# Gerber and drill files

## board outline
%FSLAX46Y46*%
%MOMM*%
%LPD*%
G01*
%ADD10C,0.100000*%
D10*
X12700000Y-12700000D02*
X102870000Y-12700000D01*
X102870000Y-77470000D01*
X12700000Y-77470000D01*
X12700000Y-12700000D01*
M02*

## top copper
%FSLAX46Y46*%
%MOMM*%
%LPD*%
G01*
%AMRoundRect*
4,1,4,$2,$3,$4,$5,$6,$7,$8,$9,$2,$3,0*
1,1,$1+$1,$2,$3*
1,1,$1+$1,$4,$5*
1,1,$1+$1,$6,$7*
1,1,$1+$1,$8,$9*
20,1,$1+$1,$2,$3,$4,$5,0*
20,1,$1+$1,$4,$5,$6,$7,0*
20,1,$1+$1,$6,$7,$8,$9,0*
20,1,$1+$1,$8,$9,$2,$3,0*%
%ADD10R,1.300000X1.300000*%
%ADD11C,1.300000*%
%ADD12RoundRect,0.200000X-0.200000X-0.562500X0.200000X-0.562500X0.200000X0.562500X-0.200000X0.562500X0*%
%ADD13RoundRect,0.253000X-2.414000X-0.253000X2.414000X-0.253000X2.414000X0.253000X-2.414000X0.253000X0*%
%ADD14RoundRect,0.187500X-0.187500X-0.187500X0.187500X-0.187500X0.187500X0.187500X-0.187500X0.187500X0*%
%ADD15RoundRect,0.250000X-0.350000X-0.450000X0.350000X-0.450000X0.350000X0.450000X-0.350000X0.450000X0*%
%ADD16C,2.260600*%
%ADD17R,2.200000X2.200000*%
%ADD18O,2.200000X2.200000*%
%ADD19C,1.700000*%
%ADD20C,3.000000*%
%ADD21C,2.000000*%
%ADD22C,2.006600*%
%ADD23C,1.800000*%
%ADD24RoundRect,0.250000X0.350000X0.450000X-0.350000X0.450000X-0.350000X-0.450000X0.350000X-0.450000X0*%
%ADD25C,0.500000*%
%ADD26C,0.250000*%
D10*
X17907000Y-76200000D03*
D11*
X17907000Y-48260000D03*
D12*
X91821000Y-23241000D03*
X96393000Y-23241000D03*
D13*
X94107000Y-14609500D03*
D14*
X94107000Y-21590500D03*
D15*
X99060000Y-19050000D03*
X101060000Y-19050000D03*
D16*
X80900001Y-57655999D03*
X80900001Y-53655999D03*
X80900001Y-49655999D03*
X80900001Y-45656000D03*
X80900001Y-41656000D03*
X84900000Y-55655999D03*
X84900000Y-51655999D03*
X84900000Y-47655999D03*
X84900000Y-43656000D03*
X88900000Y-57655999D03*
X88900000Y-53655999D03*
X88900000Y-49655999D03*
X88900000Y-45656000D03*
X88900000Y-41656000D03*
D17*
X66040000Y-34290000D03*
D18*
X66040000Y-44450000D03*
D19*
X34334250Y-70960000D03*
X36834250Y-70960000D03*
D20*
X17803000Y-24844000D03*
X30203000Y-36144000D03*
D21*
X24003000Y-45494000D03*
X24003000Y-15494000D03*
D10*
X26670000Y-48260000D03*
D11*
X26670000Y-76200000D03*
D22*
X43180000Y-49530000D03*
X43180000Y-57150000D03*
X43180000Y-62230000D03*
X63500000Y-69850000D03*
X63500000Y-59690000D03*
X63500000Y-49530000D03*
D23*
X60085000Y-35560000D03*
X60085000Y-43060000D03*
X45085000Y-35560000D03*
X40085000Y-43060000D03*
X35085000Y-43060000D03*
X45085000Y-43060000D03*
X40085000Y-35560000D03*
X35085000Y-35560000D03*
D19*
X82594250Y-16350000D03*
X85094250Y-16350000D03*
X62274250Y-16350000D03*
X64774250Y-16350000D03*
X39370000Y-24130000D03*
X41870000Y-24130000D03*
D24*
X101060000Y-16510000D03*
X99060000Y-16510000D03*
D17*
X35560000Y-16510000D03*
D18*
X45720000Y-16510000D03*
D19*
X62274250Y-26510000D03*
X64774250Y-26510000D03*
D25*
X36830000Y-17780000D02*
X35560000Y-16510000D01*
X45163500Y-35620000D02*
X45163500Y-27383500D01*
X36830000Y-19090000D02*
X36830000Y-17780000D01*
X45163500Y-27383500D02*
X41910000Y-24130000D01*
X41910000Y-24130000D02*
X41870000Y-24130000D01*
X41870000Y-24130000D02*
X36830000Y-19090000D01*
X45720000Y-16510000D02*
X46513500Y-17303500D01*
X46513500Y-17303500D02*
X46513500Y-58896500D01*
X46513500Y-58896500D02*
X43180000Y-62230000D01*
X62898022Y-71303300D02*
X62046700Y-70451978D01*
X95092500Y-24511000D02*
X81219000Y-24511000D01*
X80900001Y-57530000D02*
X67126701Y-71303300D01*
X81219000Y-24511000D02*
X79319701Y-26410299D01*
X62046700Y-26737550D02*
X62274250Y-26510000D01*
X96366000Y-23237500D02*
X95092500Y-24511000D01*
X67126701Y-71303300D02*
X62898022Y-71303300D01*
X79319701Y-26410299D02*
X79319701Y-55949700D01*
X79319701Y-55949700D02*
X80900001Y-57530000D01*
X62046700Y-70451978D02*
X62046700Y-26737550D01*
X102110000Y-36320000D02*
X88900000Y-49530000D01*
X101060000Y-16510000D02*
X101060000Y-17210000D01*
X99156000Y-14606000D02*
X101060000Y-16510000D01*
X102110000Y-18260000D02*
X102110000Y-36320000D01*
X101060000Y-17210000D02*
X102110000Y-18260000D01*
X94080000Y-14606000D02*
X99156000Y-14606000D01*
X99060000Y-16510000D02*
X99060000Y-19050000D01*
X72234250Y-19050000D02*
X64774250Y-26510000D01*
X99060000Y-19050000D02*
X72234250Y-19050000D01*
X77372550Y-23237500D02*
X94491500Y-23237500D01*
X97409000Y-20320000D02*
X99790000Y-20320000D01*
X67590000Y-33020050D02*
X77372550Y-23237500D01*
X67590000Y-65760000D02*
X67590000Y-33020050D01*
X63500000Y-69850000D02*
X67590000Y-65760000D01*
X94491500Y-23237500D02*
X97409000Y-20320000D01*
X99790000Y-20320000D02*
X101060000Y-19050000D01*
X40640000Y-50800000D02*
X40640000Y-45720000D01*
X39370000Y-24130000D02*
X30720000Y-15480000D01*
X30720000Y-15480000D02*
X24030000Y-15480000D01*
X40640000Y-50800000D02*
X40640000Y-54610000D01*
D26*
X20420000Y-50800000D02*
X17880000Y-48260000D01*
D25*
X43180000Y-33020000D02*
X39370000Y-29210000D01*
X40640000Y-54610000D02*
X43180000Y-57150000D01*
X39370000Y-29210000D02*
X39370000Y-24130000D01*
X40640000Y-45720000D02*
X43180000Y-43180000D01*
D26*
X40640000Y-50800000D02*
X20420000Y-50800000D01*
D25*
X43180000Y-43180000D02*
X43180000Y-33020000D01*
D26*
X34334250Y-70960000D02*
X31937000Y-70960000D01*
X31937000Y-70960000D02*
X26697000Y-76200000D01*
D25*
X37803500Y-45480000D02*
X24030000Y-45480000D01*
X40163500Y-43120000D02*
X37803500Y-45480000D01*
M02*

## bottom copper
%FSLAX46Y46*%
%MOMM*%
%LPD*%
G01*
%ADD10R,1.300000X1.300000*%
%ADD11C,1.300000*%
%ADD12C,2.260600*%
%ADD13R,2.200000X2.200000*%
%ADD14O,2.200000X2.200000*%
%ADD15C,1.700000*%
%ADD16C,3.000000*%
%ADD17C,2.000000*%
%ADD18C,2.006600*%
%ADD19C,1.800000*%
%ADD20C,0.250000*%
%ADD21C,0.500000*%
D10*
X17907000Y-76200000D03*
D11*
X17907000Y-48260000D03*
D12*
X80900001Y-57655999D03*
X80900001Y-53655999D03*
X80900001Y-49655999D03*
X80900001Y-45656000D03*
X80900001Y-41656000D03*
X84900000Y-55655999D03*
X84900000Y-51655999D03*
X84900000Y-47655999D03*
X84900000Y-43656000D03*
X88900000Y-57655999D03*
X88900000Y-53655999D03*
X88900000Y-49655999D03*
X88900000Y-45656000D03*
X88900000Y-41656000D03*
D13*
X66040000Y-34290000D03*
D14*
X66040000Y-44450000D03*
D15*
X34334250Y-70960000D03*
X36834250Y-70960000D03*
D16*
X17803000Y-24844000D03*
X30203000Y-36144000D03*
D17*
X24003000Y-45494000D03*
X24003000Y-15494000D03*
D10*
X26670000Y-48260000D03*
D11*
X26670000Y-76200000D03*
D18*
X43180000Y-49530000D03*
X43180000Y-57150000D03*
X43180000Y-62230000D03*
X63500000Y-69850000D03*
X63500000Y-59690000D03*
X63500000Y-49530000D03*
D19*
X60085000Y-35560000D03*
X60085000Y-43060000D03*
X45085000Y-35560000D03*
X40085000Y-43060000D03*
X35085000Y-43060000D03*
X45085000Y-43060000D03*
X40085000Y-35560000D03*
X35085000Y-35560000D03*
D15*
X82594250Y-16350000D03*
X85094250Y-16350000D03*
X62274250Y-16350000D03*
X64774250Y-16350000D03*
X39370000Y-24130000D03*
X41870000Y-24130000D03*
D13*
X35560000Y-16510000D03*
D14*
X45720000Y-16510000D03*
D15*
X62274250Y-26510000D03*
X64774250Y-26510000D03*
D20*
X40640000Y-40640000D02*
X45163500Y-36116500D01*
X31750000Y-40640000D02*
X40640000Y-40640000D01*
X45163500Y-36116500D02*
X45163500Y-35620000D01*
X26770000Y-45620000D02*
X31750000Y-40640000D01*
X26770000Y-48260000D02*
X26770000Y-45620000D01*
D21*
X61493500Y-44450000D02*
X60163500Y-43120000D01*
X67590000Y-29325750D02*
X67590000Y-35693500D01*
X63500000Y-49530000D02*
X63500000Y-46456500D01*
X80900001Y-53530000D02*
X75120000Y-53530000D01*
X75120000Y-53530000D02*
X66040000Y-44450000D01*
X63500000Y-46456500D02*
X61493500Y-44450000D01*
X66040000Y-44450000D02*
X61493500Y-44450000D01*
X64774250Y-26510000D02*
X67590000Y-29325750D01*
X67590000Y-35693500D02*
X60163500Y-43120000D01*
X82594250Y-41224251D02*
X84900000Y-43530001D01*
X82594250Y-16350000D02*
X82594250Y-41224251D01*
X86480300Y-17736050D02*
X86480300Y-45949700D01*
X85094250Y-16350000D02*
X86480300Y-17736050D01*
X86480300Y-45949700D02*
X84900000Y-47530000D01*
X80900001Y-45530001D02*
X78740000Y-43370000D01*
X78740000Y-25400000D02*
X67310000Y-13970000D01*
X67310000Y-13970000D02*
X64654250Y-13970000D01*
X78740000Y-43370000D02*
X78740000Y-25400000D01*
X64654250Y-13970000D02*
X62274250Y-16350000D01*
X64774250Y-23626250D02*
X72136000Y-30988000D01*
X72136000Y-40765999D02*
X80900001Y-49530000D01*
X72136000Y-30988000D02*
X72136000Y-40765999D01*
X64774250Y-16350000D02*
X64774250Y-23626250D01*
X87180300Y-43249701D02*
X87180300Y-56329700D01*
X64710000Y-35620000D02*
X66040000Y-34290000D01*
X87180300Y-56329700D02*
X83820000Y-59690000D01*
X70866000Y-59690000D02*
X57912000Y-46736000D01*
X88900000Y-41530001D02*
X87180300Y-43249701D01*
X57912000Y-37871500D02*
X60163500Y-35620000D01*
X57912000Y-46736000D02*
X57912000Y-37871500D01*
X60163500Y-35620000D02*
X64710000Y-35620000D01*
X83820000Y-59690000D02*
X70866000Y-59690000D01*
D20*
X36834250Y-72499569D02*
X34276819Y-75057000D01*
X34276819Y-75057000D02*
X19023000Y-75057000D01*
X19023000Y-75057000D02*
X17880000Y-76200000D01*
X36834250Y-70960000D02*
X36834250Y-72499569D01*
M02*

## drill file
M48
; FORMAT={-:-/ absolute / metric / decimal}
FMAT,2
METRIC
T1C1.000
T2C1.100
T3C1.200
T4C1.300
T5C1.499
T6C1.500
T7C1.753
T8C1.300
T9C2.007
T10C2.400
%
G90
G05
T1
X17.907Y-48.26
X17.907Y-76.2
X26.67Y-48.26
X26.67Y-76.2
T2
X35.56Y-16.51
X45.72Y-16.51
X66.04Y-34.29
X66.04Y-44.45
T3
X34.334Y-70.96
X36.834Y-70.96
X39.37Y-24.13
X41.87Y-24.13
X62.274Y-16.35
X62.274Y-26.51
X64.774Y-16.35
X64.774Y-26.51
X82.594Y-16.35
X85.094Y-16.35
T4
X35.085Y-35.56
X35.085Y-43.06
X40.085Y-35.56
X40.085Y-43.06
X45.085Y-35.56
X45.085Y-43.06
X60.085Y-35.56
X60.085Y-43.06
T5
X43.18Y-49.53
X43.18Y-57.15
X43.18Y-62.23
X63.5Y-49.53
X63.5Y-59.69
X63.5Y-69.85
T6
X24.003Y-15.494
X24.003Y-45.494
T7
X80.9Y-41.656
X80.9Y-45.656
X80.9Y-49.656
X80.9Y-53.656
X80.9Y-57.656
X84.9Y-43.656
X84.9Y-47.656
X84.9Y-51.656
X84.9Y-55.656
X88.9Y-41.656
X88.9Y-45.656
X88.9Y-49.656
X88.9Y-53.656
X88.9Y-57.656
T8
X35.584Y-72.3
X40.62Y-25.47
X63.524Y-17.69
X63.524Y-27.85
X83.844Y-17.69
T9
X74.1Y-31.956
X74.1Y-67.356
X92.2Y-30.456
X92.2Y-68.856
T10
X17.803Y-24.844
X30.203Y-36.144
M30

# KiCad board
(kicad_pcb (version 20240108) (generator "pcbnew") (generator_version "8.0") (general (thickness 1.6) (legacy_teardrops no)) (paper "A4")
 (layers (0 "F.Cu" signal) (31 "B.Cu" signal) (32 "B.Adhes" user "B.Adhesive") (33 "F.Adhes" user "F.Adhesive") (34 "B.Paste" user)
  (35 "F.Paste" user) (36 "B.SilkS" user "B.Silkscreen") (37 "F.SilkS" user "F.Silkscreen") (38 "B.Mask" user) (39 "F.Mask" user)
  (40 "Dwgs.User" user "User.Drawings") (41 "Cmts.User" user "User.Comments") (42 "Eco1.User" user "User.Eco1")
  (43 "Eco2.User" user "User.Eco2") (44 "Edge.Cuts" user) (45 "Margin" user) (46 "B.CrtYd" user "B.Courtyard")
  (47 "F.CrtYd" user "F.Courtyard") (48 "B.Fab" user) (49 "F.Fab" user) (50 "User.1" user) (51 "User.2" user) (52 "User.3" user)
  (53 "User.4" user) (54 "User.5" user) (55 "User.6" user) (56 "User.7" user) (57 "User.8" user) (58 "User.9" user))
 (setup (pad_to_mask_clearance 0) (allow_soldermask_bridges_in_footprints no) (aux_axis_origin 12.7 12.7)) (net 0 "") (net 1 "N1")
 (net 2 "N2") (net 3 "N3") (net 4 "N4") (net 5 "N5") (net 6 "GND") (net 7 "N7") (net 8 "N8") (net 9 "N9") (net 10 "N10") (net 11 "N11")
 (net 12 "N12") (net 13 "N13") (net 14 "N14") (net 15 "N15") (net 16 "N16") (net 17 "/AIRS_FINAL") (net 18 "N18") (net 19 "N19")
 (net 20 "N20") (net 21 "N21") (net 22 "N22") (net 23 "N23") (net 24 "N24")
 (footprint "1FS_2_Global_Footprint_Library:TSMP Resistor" (layer "F.Cu") (at 17.907 62.103 90)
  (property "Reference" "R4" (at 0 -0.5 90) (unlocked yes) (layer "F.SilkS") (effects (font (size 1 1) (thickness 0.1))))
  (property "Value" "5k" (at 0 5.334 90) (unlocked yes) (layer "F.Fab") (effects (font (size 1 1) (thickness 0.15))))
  (pad "1" thru_hole rect (at -14.097 0 90) (size 1.3 1.3) (drill 1) (layers "*.Cu" "*.Mask") (remove_unused_layers no) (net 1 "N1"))
  (pad "2" thru_hole circle (at 13.843 0 90) (size 1.3 1.3) (drill 1) (layers "*.Cu" "*.Mask") (remove_unused_layers no) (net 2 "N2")))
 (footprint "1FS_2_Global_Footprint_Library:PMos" (layer "F.Cu") (at 94.182 18.5485)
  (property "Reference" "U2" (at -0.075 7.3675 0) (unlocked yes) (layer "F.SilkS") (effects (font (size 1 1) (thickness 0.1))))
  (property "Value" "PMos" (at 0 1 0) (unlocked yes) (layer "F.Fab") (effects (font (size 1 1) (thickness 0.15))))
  (pad "1" smd roundrect (at -2.361 4.6925) (size 0.8 1.525) (layers "F.Cu" "F.Paste" "F.Mask") (roundrect_rratio 0.25) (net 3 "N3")
   (thermal_bridge_angle 45))
  (pad "2" smd roundrect (at 2.211 4.6925) (size 0.8 1.525) (layers "F.Cu" "F.Paste" "F.Mask") (roundrect_rratio 0.25) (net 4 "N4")
   (thermal_bridge_angle 45))
  (pad "3" smd roundrect (at -0.075 -3.939) (size 5.334 1.012) (layers "F.Cu" "F.Paste" "F.Mask") (roundrect_rratio 0.25) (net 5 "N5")
   (thermal_bridge_angle 45))
  (pad "4" smd roundrect (at -0.075 3.042) (size 0.75 0.75) (layers "F.Cu" "F.Paste" "F.Mask") (roundrect_rratio 0.25)
   (thermal_bridge_angle 45)))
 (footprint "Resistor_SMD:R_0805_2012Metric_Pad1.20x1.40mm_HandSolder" (layer "F.Cu") (at 100.06 19.05)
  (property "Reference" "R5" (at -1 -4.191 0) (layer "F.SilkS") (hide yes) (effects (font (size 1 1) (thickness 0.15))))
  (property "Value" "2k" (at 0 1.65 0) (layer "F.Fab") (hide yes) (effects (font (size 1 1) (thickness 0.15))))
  (pad "1" smd roundrect (at -1 0) (size 1.2 1.4) (layers "F.Cu" "F.Paste" "F.Mask") (roundrect_rratio 0.2083333333) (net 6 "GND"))
  (pad "2" smd roundrect (at 1 0) (size 1.2 1.4) (layers "F.Cu" "F.Paste" "F.Mask") (roundrect_rratio 0.2083333333) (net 3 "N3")))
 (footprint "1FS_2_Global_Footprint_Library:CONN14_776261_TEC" (layer "F.Cu") (at 83.9 50.9105 90)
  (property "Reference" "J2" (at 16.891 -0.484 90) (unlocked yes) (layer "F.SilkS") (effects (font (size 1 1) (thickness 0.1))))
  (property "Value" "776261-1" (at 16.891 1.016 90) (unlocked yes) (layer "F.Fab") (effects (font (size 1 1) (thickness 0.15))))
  (pad "" np_thru_hole circle (at -17.945499 8.300001 90) (size 2.0066 2.0066) (drill 2.0066) (layers "*.Cu" "*.Mask"))
  (pad "" np_thru_hole circle (at -16.445503 -9.799999 90) (size 2.0066 2.0066) (drill 2.0066) (layers "*.Cu" "*.Mask"))
  (pad "" np_thru_hole circle (at 18.954504 -9.799999 90) (size 2.0066 2.0066) (drill 2.0066) (layers "*.Cu" "*.Mask"))
  (pad "" np_thru_hole circle (at 20.454501 8.300001 90) (size 2.0066 2.0066) (drill 2.0066) (layers "*.Cu" "*.Mask"))
  (pad "1" thru_hole circle (at -6.745499 -2.999999 90) (size 2.2606 2.2606) (drill 1.7526) (layers "*.Cu" "*.Mask")
   (remove_unused_layers no) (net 4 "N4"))
  (pad "2" thru_hole circle (at -2.745499 -2.999999 90) (size 2.2606 2.2606) (drill 1.7526) (layers "*.Cu" "*.Mask")
   (remove_unused_layers no) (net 6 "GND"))
  (pad "3" thru_hole circle (at 1.254501 -2.999999 90) (size 2.2606 2.2606) (drill 1.7526) (layers "*.Cu" "*.Mask")
   (remove_unused_layers no) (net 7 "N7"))
  (pad "4" thru_hole circle (at 5.2545 -2.999999 90) (size 2.2606 2.2606) (drill 1.7526) (layers "*.Cu" "*.Mask") (remove_unused_layers no)
   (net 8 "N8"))
  (pad "5" thru_hole circle (at 9.2545 -2.999999 90) (size 2.2606 2.2606) (drill 1.7526) (layers "*.Cu" "*.Mask") (remove_unused_layers no)
   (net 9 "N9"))
  (pad "6" thru_hole circle (at -4.745499 1 90) (size 2.2606 2.2606) (drill 1.7526) (layers "*.Cu" "*.Mask") (remove_unused_layers no)
   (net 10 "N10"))
  (pad "7" thru_hole circle (at -0.745499 1 90) (size 2.2606 2.2606) (drill 1.7526) (layers "*.Cu" "*.Mask") (remove_unused_layers no)
   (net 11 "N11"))
  (pad "8" thru_hole circle (at 3.254501 1 90) (size 2.2606 2.2606) (drill 1.7526) (layers "*.Cu" "*.Mask") (remove_unused_layers no)
   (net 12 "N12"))
  (pad "9" thru_hole circle (at 7.2545 1 90) (size 2.2606 2.2606) (drill 1.7526) (layers "*.Cu" "*.Mask") (remove_unused_layers no)
   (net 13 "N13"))
  (pad "10" thru_hole circle (at -6.745499 5 90) (size 2.2606 2.2606) (drill 1.7526) (layers "*.Cu" "*.Mask") (remove_unused_layers no)
   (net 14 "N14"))
  (pad "11" thru_hole circle (at -2.745499 5 90) (size 2.2606 2.2606) (drill 1.7526) (layers "*.Cu" "*.Mask") (remove_unused_layers no)
   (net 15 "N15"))
  (pad "12" thru_hole circle (at 1.254501 5 90) (size 2.2606 2.2606) (drill 1.7526) (layers "*.Cu" "*.Mask") (remove_unused_layers no)
   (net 5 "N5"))
  (pad "13" thru_hole circle (at 5.2545 5 90) (size 2.2606 2.2606) (drill 1.7526) (layers "*.Cu" "*.Mask") (remove_unused_layers no)
   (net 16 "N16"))
  (pad "14" thru_hole circle (at 9.2545 5 90) (size 2.2606 2.2606) (drill 1.7526) (layers "*.Cu" "*.Mask") (remove_unused_layers no)
   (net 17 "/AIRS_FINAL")))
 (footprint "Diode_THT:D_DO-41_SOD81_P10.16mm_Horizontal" (layer "F.Cu") (at 66.04 34.29 -90)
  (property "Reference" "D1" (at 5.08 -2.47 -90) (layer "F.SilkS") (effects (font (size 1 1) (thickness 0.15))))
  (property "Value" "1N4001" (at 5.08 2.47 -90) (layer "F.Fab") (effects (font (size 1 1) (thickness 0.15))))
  (pad "1" thru_hole rect (at 0 0 270) (size 2.2 2.2) (drill 1.1) (layers "*.Cu" "*.Mask") (remove_unused_layers no) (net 17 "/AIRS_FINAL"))
  (pad "2" thru_hole oval (at 10.16 0 270) (size 2.2 2.2) (drill 1.1) (layers "*.Cu" "*.Mask") (remove_unused_layers no) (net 6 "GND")))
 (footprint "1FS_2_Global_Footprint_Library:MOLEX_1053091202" (layer "F.Cu") (at 34.33425 70.96)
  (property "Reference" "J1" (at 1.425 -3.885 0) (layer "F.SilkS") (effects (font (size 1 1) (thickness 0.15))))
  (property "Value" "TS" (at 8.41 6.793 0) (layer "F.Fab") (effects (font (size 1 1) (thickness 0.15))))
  (pad "" np_thru_hole circle (at 1.25 1.34) (size 1.3 1.3) (drill 1.3) (layers "*.Cu" "*.Mask"))
  (pad "1" thru_hole circle (at 0 0) (size 1.7 1.7) (drill 1.2) (layers "*.Cu") (remove_unused_layers no) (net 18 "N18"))
  (pad "2" thru_hole circle (at 2.5 0) (size 1.7 1.7) (drill 1.2) (layers "*.Cu") (remove_unused_layers no) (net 1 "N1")))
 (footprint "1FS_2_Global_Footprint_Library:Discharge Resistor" (layer "F.Cu") (at 24.003 30.357 -90)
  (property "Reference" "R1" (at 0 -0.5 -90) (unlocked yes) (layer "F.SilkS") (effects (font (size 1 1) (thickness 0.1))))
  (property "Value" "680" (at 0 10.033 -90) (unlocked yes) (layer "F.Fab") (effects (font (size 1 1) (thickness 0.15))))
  (pad "" np_thru_hole circle (at -5.513 6.2 270) (size 3 3) (drill 2.4) (layers "F&B.Cu" "*.Mask"))
  (pad "" np_thru_hole circle (at 5.787 -6.2 270) (size 3 3) (drill 2.4) (layers "F&B.Cu" "*.Mask"))
  (pad "1" thru_hole circle (at 15.137 0 270) (size 2 2) (drill 1.5) (layers "*.Cu" "*.Mask") (remove_unused_layers no) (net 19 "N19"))
  (pad "2" thru_hole circle (at -14.863 0 270) (size 2 2) (drill 1.5) (layers "*.Cu" "*.Mask") (remove_unused_layers no) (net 2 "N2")))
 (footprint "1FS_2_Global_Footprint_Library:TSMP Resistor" (layer "F.Cu") (at 26.67 62.357 -90)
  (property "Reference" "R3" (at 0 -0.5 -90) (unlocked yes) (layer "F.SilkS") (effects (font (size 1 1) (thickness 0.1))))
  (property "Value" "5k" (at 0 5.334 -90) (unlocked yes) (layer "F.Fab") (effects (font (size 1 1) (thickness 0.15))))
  (pad "1" thru_hole rect (at -14.097 0 270) (size 1.3 1.3) (drill 1) (layers "*.Cu" "*.Mask") (remove_unused_layers no) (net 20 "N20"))
  (pad "2" thru_hole circle (at 13.843 0 270) (size 1.3 1.3) (drill 1) (layers "*.Cu" "*.Mask") (remove_unused_layers no) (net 18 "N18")))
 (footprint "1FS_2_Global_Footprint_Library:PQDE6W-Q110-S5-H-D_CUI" (layer "F.Cu") (at 43.18 49.53)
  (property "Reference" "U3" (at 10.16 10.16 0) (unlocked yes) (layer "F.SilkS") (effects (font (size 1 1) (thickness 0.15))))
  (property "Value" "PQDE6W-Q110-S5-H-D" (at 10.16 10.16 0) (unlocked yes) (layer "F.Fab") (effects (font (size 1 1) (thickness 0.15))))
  (pad "1" thru_hole circle (at 0 0) (size 2.0066 2.0066) (drill 1.4986) (layers "*.Cu" "*.Mask") (remove_unused_layers no) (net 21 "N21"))
  (pad "2" thru_hole circle (at 0 7.62) (size 2.0066 2.0066) (drill 1.4986) (layers "*.Cu" "*.Mask") (remove_unused_layers no) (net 2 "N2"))
  (pad "3" thru_hole circle (at 0 12.7) (size 2.0066 2.0066) (drill 1.4986) (layers "*.Cu" "*.Mask") (remove_unused_layers no)
   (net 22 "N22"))
  (pad "4" thru_hole circle (at 20.32 20.32) (size 2.0066 2.0066) (drill 1.4986) (layers "*.Cu" "*.Mask") (remove_unused_layers no)
   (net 3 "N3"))
  (pad "5" thru_hole circle (at 20.32 10.16) (size 2.0066 2.0066) (drill 1.4986) (layers "*.Cu" "*.Mask") (remove_unused_layers no)
   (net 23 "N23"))
  (pad "6" thru_hole circle (at 20.32 0) (size 2.0066 2.0066) (drill 1.4986) (layers "*.Cu" "*.Mask") (remove_unused_layers no)
   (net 6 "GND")))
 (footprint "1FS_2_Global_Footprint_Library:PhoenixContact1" (layer "F.Cu") (at 44.5 39.41 -90)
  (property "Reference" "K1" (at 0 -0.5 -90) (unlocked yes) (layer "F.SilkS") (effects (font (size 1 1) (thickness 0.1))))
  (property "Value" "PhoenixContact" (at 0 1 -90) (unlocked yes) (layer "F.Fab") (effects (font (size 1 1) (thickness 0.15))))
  (pad "1" thru_hole circle (at -3.85 -15.585 270) (size 1.8 1.8) (drill 1.3) (layers "*.Cu" "*.Mask") (remove_unused_layers no)
   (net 17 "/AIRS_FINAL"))
  (pad "2" thru_hole circle (at 3.65 -15.585 270) (size 1.8 1.8) (drill 1.3) (layers "*.Cu" "*.Mask") (remove_unused_layers no)
   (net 6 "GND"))
  (pad "3" thru_hole circle (at -3.85 -0.585 270) (size 1.8 1.8) (drill 1.3) (layers "*.Cu" "*.Mask") (remove_unused_layers no)
   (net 20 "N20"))
  (pad "4" thru_hole circle (at 3.65 4.415 270) (size 1.8 1.8) (drill 1.3) (layers "*.Cu" "*.Mask") (remove_unused_layers no) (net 19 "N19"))
  (pad "5" thru_hole circle (at 3.65 9.415 270) (size 1.8 1.8) (drill 1.3) (layers "*.Cu" "*.Mask") (remove_unused_layers no) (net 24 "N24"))
  (pad "6" thru_hole circle (at 3.65 -0.585 270) (size 1.8 1.8) (drill 1.3) (layers "*.Cu" "*.Mask") (remove_unused_layers no))
  (pad "7" thru_hole circle (at -3.85 4.415 270) (size 1.8 1.8) (drill 1.3) (layers "*.Cu" "*.Mask") (remove_unused_layers no))
  (pad "8" thru_hole circle (at -3.85 9.415 270) (size 1.8 1.8) (drill 1.3) (layers "*.Cu" "*.Mask") (remove_unused_layers no)))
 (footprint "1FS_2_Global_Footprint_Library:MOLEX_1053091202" (layer "F.Cu") (at 82.59425 16.35)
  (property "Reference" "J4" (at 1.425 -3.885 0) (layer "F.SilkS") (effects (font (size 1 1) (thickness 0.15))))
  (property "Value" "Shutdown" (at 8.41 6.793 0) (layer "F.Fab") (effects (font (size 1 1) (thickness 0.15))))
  (pad "" np_thru_hole circle (at 1.25 1.34) (size 1.3 1.3) (drill 1.3) (layers "*.Cu" "*.Mask"))
  (pad "1" thru_hole circle (at 0 0) (size 1.7 1.7) (drill 1.2) (layers "*.Cu") (remove_unused_layers no) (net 13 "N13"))
  (pad "2" thru_hole circle (at 2.5 0) (size 1.7 1.7) (drill 1.2) (layers "*.Cu") (remove_unused_layers no) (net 12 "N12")))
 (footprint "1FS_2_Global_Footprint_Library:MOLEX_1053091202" (layer "F.Cu") (at 62.27425 16.35)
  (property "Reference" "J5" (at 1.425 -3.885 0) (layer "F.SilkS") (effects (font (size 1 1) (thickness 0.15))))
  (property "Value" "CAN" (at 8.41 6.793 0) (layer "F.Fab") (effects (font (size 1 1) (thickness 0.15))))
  (pad "" np_thru_hole circle (at 1.25 1.34) (size 1.3 1.3) (drill 1.3) (layers "*.Cu" "*.Mask"))
  (pad "1" thru_hole circle (at 0 0) (size 1.7 1.7) (drill 1.2) (layers "*.Cu") (remove_unused_layers no) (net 8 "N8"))
  (pad "2" thru_hole circle (at 2.5 0) (size 1.7 1.7) (drill 1.2) (layers "*.Cu") (remove_unused_layers no) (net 7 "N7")))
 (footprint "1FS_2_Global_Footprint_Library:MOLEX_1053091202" (layer "F.Cu") (at 39.37 24.13)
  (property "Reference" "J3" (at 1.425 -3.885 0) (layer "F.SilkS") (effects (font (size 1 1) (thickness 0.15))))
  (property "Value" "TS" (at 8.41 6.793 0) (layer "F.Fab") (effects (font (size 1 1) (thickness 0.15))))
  (pad "" np_thru_hole circle (at 1.25 1.34) (size 1.3 1.3) (drill 1.3) (layers "*.Cu" "*.Mask"))
  (pad "1" thru_hole circle (at 0 0) (size 1.7 1.7) (drill 1.2) (layers "*.Cu") (remove_unused_layers no) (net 2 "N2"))
  (pad "2" thru_hole circle (at 2.5 0) (size 1.7 1.7) (drill 1.2) (layers "*.Cu") (remove_unused_layers no) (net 20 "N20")))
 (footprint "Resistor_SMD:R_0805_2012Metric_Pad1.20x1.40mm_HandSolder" (layer "F.Cu") (at 100.06 16.51 180)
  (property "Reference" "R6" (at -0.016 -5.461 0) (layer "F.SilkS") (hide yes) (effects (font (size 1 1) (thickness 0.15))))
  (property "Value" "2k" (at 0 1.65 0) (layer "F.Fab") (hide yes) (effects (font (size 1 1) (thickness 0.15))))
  (pad "1" smd roundrect (at -1 0 180) (size 1.2 1.4) (layers "F.Cu" "F.Paste" "F.Mask") (roundrect_rratio 0.2083333333) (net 5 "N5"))
  (pad "2" smd roundrect (at 1 0 180) (size 1.2 1.4) (layers "F.Cu" "F.Paste" "F.Mask") (roundrect_rratio 0.2083333333) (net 6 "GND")))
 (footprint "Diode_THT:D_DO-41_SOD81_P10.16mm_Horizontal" (layer "F.Cu") (at 35.56 16.51)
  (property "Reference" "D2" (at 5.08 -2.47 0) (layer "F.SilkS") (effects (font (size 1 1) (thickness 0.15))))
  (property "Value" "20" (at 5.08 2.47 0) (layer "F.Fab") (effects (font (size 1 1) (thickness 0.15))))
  (pad "1" thru_hole rect (at 0 0) (size 2.2 2.2) (drill 1.1) (layers "*.Cu" "*.Mask") (remove_unused_layers no) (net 20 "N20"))
  (pad "2" thru_hole oval (at 10.16 0) (size 2.2 2.2) (drill 1.1) (layers "*.Cu" "*.Mask") (remove_unused_layers no) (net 22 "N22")))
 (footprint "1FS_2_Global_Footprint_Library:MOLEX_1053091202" (layer "F.Cu") (at 62.27425 26.51)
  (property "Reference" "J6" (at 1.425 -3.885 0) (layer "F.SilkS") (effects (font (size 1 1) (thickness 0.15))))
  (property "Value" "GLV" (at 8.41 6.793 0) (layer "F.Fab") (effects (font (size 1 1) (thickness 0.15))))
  (pad "" np_thru_hole circle (at 1.25 1.34) (size 1.3 1.3) (drill 1.3) (layers "*.Cu" "*.Mask"))
  (pad "1" thru_hole circle (at 0 0) (size 1.7 1.7) (drill 1.2) (layers "*.Cu") (remove_unused_layers no) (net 4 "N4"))
  (pad "2" thru_hole circle (at 2.5 0) (size 1.7 1.7) (drill 1.2) (layers "*.Cu") (remove_unused_layers no) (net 6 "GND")))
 (gr_rect (start 12.7 12.7) (end 102.87 77.47) (stroke (width 0.1) (type default)) (fill none) (layer "Edge.Cuts"))
 (segment (start 36.83 17.78) (end 35.56 16.51) (width 0.5) (layer "F.Cu") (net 20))
 (segment (start 45.1635 35.62) (end 45.1635 27.3835) (width 0.5) (layer "F.Cu") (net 20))
 (segment (start 36.83 19.09) (end 36.83 17.78) (width 0.5) (layer "F.Cu") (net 20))
 (segment (start 45.1635 27.3835) (end 41.91 24.13) (width 0.5) (layer "F.Cu") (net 20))
 (segment (start 41.91 24.13) (end 41.87 24.13) (width 0.5) (layer "F.Cu") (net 20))
 (segment (start 41.87 24.13) (end 36.83 19.09) (width 0.5) (layer "F.Cu") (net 20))
 (segment (start 40.64 40.64) (end 45.1635 36.1165) (width 0.25) (layer "B.Cu") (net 20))
 (segment (start 31.75 40.64) (end 40.64 40.64) (width 0.25) (layer "B.Cu") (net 20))
 (segment (start 45.1635 36.1165) (end 45.1635 35.62) (width 0.25) (layer "B.Cu") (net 20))
 (segment (start 26.77 45.62) (end 31.75 40.64) (width 0.25) (layer "B.Cu") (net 20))
 (segment (start 26.77 48.26) (end 26.77 45.62) (width 0.25) (layer "B.Cu") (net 20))
 (segment (start 45.72 16.51) (end 46.5135 17.3035) (width 0.5) (layer "F.Cu") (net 22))
 (segment (start 46.5135 17.3035) (end 46.5135 58.8965) (width 0.5) (layer "F.Cu") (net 22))
 (segment (start 46.5135 58.8965) (end 43.18 62.23) (width 0.5) (layer "F.Cu") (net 22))
 (segment (start 62.898022 71.3033) (end 62.0467 70.451978) (width 0.5) (layer "F.Cu") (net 4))
 (segment (start 95.0925 24.511) (end 81.219 24.511) (width 0.5) (layer "F.Cu") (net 4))
 (segment (start 80.900001 57.53) (end 67.126701 71.3033) (width 0.5) (layer "F.Cu") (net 4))
 (segment (start 81.219 24.511) (end 79.319701 26.410299) (width 0.5) (layer "F.Cu") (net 4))
 (segment (start 62.0467 26.73755) (end 62.27425 26.51) (width 0.5) (layer "F.Cu") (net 4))
 (segment (start 96.366 23.2375) (end 95.0925 24.511) (width 0.5) (layer "F.Cu") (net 4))
 (segment (start 67.126701 71.3033) (end 62.898022 71.3033) (width 0.5) (layer "F.Cu") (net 4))
 (segment (start 79.319701 26.410299) (end 79.319701 55.9497) (width 0.5) (layer "F.Cu") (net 4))
 (segment (start 79.319701 55.9497) (end 80.900001 57.53) (width 0.5) (layer "F.Cu") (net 4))
 (segment (start 62.0467 70.451978) (end 62.0467 26.73755) (width 0.5) (layer "F.Cu") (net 4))
 (segment (start 102.11 36.32) (end 88.9 49.53) (width 0.5) (layer "F.Cu") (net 5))
 (segment (start 101.06 16.51) (end 101.06 17.21) (width 0.5) (layer "F.Cu") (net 5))
 (segment (start 99.156 14.606) (end 101.06 16.51) (width 0.5) (layer "F.Cu") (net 5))
 (segment (start 102.11 18.26) (end 102.11 36.32) (width 0.5) (layer "F.Cu") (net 5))
 (segment (start 101.06 17.21) (end 102.11 18.26) (width 0.5) (layer "F.Cu") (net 5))
 (segment (start 94.08 14.606) (end 99.156 14.606) (width 0.5) (layer "F.Cu") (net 5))
 (segment (start 99.06 16.51) (end 99.06 19.05) (width 0.5) (layer "F.Cu") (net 6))
 (segment (start 72.23425 19.05) (end 64.77425 26.51) (width 0.5) (layer "F.Cu") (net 6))
 (segment (start 99.06 19.05) (end 72.23425 19.05) (width 0.5) (layer "F.Cu") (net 6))
 (segment (start 61.4935 44.45) (end 60.1635 43.12) (width 0.5) (layer "B.Cu") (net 6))
 (segment (start 67.59 29.32575) (end 67.59 35.6935) (width 0.5) (layer "B.Cu") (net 6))
 (segment (start 63.5 49.53) (end 63.5 46.4565) (width 0.5) (layer "B.Cu") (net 6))
 (segment (start 80.900001 53.53) (end 75.12 53.53) (width 0.5) (layer "B.Cu") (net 6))
 (segment (start 75.12 53.53) (end 66.04 44.45) (width 0.5) (layer "B.Cu") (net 6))
 (segment (start 63.5 46.4565) (end 61.4935 44.45) (width 0.5) (layer "B.Cu") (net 6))
 (segment (start 66.04 44.45) (end 61.4935 44.45) (width 0.5) (layer "B.Cu") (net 6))
 (segment (start 64.77425 26.51) (end 67.59 29.32575) (width 0.5) (layer "B.Cu") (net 6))
 (segment (start 67.59 35.6935) (end 60.1635 43.12) (width 0.5) (layer "B.Cu") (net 6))
 (segment (start 77.37255 23.2375) (end 94.4915 23.2375) (width 0.5) (layer "F.Cu") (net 3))
 (segment (start 97.409 20.32) (end 99.79 20.32) (width 0.5) (layer "F.Cu") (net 3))
 (segment (start 67.59 33.02005) (end 77.37255 23.2375) (width 0.5) (layer "F.Cu") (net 3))
 (segment (start 67.59 65.76) (end 67.59 33.02005) (width 0.5) (layer "F.Cu") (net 3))
 (segment (start 63.5 69.85) (end 67.59 65.76) (width 0.5) (layer "F.Cu") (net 3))
 (segment (start 94.4915 23.2375) (end 97.409 20.32) (width 0.5) (layer "F.Cu") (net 3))
 (segment (start 99.79 20.32) (end 101.06 19.05) (width 0.5) (layer "F.Cu") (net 3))
 (segment (start 40.64 50.8) (end 40.64 45.72) (width 0.5) (layer "F.Cu") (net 2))
 (segment (start 39.37 24.13) (end 30.72 15.48) (width 0.5) (layer "F.Cu") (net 2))
 (segment (start 30.72 15.48) (end 24.03 15.48) (width 0.5) (layer "F.Cu") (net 2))
 (segment (start 40.64 50.8) (end 40.64 54.61) (width 0.5) (layer "F.Cu") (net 2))
 (segment (start 20.42 50.8) (end 17.88 48.26) (width 0.25) (layer "F.Cu") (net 2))
 (segment (start 43.18 33.02) (end 39.37 29.21) (width 0.5) (layer "F.Cu") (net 2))
 (segment (start 40.64 54.61) (end 43.18 57.15) (width 0.5) (layer "F.Cu") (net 2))
 (segment (start 39.37 29.21) (end 39.37 24.13) (width 0.5) (layer "F.Cu") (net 2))
 (segment (start 40.64 45.72) (end 43.18 43.18) (width 0.5) (layer "F.Cu") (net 2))
 (segment (start 40.64 50.8) (end 20.42 50.8) (width 0.25) (layer "F.Cu") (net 2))
 (segment (start 43.18 43.18) (end 43.18 33.02) (width 0.5) (layer "F.Cu") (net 2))
 (segment (start 82.59425 41.224251) (end 84.9 43.530001) (width 0.5) (layer "B.Cu") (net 13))
 (segment (start 82.59425 16.35) (end 82.59425 41.224251) (width 0.5) (layer "B.Cu") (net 13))
 (segment (start 86.4803 17.73605) (end 86.4803 45.9497) (width 0.5) (layer "B.Cu") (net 12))
 (segment (start 85.09425 16.35) (end 86.4803 17.73605) (width 0.5) (layer "B.Cu") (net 12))
 (segment (start 86.4803 45.9497) (end 84.9 47.53) (width 0.5) (layer "B.Cu") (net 12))
 (segment (start 80.900001 45.530001) (end 78.74 43.37) (width 0.5) (layer "B.Cu") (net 8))
 (segment (start 78.74 25.4) (end 67.31 13.97) (width 0.5) (layer "B.Cu") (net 8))
 (segment (start 67.31 13.97) (end 64.65425 13.97) (width 0.5) (layer "B.Cu") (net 8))
 (segment (start 78.74 43.37) (end 78.74 25.4) (width 0.5) (layer "B.Cu") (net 8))
 (segment (start 64.65425 13.97) (end 62.27425 16.35) (width 0.5) (layer "B.Cu") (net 8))
 (segment (start 64.77425 23.62625) (end 72.136 30.988) (width 0.5) (layer "B.Cu") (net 7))
 (segment (start 72.136 40.765999) (end 80.900001 49.53) (width 0.5) (layer "B.Cu") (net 7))
 (segment (start 72.136 30.988) (end 72.136 40.765999) (width 0.5) (layer "B.Cu") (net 7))
 (segment (start 64.77425 16.35) (end 64.77425 23.62625) (width 0.5) (layer "B.Cu") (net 7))
 (segment (start 87.1803 43.249701) (end 87.1803 56.3297) (width 0.5) (layer "B.Cu") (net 17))
 (segment (start 64.71 35.62) (end 66.04 34.29) (width 0.5) (layer "B.Cu") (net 17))
 (segment (start 87.1803 56.3297) (end 83.82 59.69) (width 0.5) (layer "B.Cu") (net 17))
 (segment (start 70.866 59.69) (end 57.912 46.736) (width 0.5) (layer "B.Cu") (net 17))
 (segment (start 88.9 41.530001) (end 87.1803 43.249701) (width 0.5) (layer "B.Cu") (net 17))
 (segment (start 57.912 37.8715) (end 60.1635 35.62) (width 0.5) (layer "B.Cu") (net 17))
 (segment (start 57.912 46.736) (end 57.912 37.8715) (width 0.5) (layer "B.Cu") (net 17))
 (segment (start 60.1635 35.62) (end 64.71 35.62) (width 0.5) (layer "B.Cu") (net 17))
 (segment (start 83.82 59.69) (end 70.866 59.69) (width 0.5) (layer "B.Cu") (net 17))
 (segment (start 34.33425 70.96) (end 31.937 70.96) (width 0.25) (layer "F.Cu") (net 18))
 (segment (start 31.937 70.96) (end 26.697 76.2) (width 0.25) (layer "F.Cu") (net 18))
 (segment (start 36.83425 72.499569) (end 34.276819 75.057) (width 0.25) (layer "B.Cu") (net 1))
 (segment (start 34.276819 75.057) (end 19.023 75.057) (width 0.25) (layer "B.Cu") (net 1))
 (segment (start 19.023 75.057) (end 17.88 76.2) (width 0.25) (layer "B.Cu") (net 1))
 (segment (start 36.83425 70.96) (end 36.83425 72.499569) (width 0.25) (layer "B.Cu") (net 1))
 (segment (start 37.8035 45.48) (end 24.03 45.48) (width 0.5) (layer "F.Cu") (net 19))
 (segment (start 40.1635 43.12) (end 37.8035 45.48) (width 0.5) (layer "F.Cu") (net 19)))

